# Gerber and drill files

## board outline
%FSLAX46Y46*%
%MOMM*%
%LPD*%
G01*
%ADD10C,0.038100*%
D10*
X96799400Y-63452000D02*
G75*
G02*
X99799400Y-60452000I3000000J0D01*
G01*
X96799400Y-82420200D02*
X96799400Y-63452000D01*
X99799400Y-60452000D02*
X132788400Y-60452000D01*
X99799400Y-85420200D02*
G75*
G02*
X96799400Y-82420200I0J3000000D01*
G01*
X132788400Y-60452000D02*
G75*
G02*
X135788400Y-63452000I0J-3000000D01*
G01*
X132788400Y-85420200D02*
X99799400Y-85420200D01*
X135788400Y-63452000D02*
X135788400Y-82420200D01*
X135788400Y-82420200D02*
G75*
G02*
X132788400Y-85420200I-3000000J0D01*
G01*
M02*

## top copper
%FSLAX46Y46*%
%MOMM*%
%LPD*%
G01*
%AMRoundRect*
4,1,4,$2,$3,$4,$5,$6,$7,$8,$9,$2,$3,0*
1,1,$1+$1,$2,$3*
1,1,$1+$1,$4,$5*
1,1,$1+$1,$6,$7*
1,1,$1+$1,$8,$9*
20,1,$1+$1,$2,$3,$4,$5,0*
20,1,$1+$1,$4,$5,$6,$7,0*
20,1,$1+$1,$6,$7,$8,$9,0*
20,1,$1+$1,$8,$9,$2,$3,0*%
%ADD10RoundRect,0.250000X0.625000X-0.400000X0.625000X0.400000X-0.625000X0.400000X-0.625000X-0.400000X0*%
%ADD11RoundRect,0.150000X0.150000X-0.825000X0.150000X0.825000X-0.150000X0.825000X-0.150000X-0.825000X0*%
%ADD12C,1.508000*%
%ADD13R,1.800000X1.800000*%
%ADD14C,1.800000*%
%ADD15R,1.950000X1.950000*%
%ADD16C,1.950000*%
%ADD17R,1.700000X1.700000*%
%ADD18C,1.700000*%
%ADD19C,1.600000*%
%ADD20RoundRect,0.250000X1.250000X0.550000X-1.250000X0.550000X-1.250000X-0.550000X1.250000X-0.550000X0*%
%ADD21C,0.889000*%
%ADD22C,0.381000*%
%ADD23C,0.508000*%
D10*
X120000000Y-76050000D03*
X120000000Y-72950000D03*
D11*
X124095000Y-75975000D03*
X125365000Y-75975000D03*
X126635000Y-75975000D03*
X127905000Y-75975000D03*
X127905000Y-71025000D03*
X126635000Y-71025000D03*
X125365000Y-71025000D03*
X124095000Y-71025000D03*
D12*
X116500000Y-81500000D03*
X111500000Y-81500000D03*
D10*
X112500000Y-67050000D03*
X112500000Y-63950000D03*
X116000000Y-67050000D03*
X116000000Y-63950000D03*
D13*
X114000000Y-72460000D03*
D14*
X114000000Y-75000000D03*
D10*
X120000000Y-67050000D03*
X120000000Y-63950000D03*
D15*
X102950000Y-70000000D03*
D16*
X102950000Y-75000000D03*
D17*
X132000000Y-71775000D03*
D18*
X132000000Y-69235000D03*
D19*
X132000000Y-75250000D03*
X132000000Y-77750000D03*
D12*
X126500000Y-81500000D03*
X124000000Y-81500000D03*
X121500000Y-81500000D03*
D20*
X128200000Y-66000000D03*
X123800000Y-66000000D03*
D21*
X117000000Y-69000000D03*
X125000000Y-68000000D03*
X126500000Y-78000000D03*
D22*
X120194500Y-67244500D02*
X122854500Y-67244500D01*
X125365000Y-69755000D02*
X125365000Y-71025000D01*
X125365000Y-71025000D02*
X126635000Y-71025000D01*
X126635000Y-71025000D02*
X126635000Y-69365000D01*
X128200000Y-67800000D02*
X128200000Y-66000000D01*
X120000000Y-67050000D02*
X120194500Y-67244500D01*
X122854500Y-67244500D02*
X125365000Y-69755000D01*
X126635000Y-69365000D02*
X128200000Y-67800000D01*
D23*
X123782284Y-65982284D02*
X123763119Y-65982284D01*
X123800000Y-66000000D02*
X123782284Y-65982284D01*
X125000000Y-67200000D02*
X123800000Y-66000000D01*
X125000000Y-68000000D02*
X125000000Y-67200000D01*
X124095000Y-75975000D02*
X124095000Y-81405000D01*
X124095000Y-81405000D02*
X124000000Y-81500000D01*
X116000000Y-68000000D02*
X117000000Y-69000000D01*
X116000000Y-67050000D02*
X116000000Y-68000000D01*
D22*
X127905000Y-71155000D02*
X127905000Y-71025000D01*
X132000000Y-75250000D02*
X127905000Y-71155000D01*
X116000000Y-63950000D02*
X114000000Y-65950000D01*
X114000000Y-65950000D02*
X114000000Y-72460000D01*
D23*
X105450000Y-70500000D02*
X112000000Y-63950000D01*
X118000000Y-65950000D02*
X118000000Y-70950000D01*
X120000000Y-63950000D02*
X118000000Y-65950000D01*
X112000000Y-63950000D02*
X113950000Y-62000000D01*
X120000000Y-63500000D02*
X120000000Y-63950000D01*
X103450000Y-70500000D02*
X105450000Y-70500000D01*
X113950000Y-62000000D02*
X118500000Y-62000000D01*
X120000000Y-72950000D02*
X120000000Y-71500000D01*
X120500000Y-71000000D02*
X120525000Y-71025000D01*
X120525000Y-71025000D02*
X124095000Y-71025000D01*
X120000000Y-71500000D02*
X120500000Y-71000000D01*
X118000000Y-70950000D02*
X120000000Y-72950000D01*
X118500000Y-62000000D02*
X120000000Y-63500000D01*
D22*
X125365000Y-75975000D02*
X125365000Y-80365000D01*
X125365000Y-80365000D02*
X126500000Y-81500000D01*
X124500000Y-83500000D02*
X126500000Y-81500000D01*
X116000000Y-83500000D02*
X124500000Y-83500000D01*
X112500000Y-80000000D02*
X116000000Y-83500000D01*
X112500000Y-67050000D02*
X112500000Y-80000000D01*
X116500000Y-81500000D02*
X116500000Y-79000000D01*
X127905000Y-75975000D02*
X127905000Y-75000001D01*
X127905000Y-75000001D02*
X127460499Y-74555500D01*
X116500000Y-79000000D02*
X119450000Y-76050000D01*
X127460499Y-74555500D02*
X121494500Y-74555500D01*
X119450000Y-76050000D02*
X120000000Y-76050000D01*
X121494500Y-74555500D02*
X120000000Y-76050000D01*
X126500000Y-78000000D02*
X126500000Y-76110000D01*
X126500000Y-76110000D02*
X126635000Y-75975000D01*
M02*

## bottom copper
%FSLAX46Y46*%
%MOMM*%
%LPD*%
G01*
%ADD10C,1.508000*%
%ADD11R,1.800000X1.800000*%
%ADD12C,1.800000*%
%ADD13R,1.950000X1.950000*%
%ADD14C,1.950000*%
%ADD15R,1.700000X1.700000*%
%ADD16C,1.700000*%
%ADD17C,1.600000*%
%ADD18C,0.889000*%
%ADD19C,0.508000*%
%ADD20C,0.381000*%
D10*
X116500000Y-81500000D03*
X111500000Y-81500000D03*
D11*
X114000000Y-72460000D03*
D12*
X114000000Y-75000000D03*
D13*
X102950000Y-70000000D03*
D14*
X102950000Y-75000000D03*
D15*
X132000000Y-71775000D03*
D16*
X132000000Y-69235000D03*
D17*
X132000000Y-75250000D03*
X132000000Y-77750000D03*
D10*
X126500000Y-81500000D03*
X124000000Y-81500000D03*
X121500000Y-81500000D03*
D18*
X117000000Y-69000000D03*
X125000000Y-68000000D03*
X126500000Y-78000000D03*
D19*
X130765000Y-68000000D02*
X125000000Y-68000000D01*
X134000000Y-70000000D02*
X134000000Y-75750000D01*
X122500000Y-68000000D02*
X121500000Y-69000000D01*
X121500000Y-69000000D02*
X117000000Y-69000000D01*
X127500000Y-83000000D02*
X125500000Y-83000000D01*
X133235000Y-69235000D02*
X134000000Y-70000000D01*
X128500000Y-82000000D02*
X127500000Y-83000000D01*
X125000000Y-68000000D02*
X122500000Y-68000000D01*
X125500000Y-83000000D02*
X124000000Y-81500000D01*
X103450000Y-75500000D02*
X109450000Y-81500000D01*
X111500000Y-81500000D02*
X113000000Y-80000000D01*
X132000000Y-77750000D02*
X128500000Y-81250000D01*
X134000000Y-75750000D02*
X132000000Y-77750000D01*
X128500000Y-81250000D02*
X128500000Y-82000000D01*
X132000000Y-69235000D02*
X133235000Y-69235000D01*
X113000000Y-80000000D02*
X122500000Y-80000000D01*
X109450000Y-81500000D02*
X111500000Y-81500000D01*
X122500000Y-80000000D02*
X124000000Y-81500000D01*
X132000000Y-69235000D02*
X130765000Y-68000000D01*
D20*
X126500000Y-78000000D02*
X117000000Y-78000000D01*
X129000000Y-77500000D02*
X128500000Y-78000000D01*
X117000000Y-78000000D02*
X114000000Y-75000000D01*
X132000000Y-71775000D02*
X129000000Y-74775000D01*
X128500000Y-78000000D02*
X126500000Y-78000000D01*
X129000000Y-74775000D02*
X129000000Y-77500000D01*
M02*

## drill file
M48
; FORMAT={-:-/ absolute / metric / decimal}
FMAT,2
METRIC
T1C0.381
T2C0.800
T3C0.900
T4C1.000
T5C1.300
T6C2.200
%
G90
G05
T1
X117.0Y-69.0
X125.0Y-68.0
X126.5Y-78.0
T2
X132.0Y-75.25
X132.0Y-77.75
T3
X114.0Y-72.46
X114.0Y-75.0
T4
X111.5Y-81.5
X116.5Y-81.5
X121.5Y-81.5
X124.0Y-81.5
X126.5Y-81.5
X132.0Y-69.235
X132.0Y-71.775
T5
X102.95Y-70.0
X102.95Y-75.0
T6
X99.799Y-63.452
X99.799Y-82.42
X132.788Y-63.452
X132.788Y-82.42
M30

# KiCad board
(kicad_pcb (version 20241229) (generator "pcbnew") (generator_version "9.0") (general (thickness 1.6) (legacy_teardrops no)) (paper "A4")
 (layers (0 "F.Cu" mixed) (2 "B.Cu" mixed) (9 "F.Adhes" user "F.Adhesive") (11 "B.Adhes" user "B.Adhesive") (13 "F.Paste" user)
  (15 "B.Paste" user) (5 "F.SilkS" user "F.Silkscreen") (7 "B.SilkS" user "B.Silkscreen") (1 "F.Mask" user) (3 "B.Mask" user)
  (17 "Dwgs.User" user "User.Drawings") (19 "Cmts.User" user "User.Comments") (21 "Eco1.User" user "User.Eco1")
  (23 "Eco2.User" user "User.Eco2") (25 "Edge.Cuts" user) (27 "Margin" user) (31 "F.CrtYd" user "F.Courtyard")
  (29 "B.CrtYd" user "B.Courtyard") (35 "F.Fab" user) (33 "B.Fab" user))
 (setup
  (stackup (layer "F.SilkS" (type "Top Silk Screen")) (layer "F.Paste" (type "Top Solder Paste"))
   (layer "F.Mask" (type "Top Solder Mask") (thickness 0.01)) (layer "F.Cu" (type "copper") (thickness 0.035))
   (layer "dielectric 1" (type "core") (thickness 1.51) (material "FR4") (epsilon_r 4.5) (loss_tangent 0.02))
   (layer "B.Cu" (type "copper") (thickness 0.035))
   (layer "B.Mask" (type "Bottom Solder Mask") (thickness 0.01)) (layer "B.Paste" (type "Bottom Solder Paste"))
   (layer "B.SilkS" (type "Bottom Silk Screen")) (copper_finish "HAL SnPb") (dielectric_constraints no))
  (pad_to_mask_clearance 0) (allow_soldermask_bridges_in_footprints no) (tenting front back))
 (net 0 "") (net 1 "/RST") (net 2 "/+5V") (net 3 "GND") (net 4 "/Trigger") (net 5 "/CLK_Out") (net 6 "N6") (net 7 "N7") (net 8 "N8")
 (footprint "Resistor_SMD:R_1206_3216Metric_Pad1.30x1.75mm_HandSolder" (layer "F.Cu") (at 120 74.5 90)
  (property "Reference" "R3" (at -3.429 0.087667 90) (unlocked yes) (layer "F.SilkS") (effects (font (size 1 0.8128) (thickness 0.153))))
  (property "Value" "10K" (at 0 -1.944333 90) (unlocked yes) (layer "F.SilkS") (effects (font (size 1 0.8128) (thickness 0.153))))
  (pad "1" smd roundrect (at -1.55 0 90) (size 1.3 1.75) (layers "F.Cu" "F.Mask" "F.Paste") (roundrect_rratio 0.192308) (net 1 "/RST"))
  (pad "2" smd roundrect (at 1.55 0 90) (size 1.3 1.75) (layers "F.Cu" "F.Mask" "F.Paste") (roundrect_rratio 0.192308) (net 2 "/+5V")))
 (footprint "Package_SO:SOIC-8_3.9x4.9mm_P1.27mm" (layer "F.Cu") (at 126 73.5 90)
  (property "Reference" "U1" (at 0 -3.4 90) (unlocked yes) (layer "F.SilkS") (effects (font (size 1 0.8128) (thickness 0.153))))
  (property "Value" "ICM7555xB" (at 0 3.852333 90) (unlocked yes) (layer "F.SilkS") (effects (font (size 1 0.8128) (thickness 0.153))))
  (pad "1" smd roundrect (at -2.475 -1.905 90) (size 1.95 0.6) (layers "F.Cu" "F.Mask" "F.Paste") (roundrect_rratio 0.25) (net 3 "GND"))
  (pad "2" smd roundrect (at -2.475 -0.635 90) (size 1.95 0.6) (layers "F.Cu" "F.Mask" "F.Paste") (roundrect_rratio 0.25) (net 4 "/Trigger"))
  (pad "3" smd roundrect (at -2.475 0.635 90) (size 1.95 0.6) (layers "F.Cu" "F.Mask" "F.Paste") (roundrect_rratio 0.25) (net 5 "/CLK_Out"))
  (pad "4" smd roundrect (at -2.475 1.905 90) (size 1.95 0.6) (layers "F.Cu" "F.Mask" "F.Paste") (roundrect_rratio 0.25) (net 1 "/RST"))
  (pad "5" smd roundrect (at 2.475 1.905 90) (size 1.95 0.6) (layers "F.Cu" "F.Mask" "F.Paste") (roundrect_rratio 0.25) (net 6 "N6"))
  (pad "6" smd roundrect (at 2.475 0.635 90) (size 1.95 0.6) (layers "F.Cu" "F.Mask" "F.Paste") (roundrect_rratio 0.25) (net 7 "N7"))
  (pad "7" smd roundrect (at 2.475 -0.635 90) (size 1.95 0.6) (layers "F.Cu" "F.Mask" "F.Paste") (roundrect_rratio 0.25) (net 7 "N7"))
  (pad "8" smd roundrect (at 2.475 -1.905 90) (size 1.95 0.6) (layers "F.Cu" "F.Mask" "F.Paste") (roundrect_rratio 0.25) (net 2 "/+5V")))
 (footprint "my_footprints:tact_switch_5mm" (layer "F.Cu") (at 114 81.5 180)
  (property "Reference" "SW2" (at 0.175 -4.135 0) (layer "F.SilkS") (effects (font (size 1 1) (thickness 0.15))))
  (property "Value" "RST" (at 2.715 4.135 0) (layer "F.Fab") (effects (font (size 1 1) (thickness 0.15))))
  (pad "1" thru_hole circle (at -2.5 0 180) (size 1.508 1.508) (drill 1) (layers "*.Cu" "*.Mask") (remove_unused_layers no) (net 1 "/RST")
   (solder_mask_margin 0.102))
  (pad "2" thru_hole circle (at 2.5 0 180) (size 1.508 1.508) (drill 1) (layers "*.Cu" "*.Mask") (remove_unused_layers no) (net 3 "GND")
   (solder_mask_margin 0.102)))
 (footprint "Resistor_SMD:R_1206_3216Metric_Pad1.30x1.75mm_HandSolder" (layer "F.Cu") (at 112.5 65.5 90)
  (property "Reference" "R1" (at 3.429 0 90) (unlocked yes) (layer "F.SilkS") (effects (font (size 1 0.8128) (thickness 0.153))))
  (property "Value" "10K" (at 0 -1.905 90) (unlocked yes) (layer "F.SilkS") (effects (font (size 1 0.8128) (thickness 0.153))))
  (pad "1" smd roundrect (at -1.55 0 90) (size 1.3 1.75) (layers "F.Cu" "F.Mask" "F.Paste") (roundrect_rratio 0.192308) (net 4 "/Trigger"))
  (pad "2" smd roundrect (at 1.55 0 90) (size 1.3 1.75) (layers "F.Cu" "F.Mask" "F.Paste") (roundrect_rratio 0.192308) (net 2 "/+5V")))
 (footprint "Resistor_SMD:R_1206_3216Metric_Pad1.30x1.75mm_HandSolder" (layer "F.Cu") (at 116 65.5 90)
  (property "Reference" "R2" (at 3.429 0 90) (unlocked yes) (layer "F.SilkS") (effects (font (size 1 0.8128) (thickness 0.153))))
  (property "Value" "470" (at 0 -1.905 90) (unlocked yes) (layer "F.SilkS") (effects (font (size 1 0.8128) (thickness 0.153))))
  (pad "1" smd roundrect (at -1.55 0 90) (size 1.3 1.75) (layers "F.Cu" "F.Mask" "F.Paste") (roundrect_rratio 0.192308) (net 3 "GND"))
  (pad "2" smd roundrect (at 1.55 0 90) (size 1.3 1.75) (layers "F.Cu" "F.Mask" "F.Paste") (roundrect_rratio 0.192308) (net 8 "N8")))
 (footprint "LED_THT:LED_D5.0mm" (layer "F.Cu") (at 114 72.46 -90)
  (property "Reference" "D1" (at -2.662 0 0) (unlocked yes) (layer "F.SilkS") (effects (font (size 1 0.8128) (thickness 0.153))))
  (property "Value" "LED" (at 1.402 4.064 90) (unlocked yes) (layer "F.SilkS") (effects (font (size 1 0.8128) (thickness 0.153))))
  (pad "1" thru_hole rect (at 0 0 270) (size 1.8 1.8) (drill 0.9) (layers "*.Cu" "*.Mask") (remove_unused_layers no) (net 8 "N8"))
  (pad "2" thru_hole circle (at 2.54 0 270) (size 1.8 1.8) (drill 0.9) (layers "*.Cu" "*.Mask") (remove_unused_layers no) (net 5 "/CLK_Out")))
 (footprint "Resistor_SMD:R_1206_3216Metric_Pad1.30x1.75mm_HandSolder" (layer "F.Cu") (at 120 65.5 90)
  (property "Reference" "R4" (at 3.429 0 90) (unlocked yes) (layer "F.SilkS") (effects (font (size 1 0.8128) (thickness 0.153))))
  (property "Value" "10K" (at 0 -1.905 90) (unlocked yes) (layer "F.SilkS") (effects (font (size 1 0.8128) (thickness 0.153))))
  (pad "1" smd roundrect (at -1.55 0 90) (size 1.3 1.75) (layers "F.Cu" "F.Mask" "F.Paste") (roundrect_rratio 0.192308) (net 7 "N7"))
  (pad "2" smd roundrect (at 1.55 0 90) (size 1.3 1.75) (layers "F.Cu" "F.Mask" "F.Paste") (roundrect_rratio 0.192308) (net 2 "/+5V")))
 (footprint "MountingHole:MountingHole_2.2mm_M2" (layer "F.Cu") (at 99.7994 63.452)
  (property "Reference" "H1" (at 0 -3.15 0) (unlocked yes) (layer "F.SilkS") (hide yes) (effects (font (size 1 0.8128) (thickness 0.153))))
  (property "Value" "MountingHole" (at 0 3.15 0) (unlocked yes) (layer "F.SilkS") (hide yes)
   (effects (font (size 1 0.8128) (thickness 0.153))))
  (pad "" np_thru_hole circle (at 0 0) (size 2.2 2.2) (drill 2.2) (layers "*.Cu" "*.Mask")))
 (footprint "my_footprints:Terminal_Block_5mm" (layer "F.Cu") (at 102.95 72.5 -90)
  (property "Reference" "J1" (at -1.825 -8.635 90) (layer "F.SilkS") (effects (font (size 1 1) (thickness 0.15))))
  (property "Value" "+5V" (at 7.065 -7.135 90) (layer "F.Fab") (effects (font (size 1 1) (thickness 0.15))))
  (pad "1" thru_hole rect (at -2.5 0 270) (size 1.95 1.95) (drill 1.3) (layers "*.Cu" "*.Mask") (remove_unused_layers no) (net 2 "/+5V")
   (solder_mask_margin 0.102))
  (pad "2" thru_hole circle (at 2.5 0 270) (size 1.95 1.95) (drill 1.3) (layers "*.Cu" "*.Mask") (remove_unused_layers no) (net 3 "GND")
   (solder_mask_margin 0.102)))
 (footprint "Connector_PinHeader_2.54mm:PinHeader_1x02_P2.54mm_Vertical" (layer "F.Cu") (at 132 71.775 180)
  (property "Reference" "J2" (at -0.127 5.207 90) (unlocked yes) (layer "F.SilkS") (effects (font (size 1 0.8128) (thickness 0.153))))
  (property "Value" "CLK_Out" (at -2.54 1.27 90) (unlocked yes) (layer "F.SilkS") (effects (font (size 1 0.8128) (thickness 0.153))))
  (pad "1" thru_hole rect (at 0 0 180) (size 1.7 1.7) (drill 1) (layers "*.Cu" "*.Mask") (remove_unused_layers no) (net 5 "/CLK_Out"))
  (pad "2" thru_hole circle (at 0 2.54 180) (size 1.7 1.7) (drill 1) (layers "*.Cu" "*.Mask") (remove_unused_layers no) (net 3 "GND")))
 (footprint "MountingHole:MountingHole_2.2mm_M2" (layer "F.Cu") (at 132.7884 82.4202)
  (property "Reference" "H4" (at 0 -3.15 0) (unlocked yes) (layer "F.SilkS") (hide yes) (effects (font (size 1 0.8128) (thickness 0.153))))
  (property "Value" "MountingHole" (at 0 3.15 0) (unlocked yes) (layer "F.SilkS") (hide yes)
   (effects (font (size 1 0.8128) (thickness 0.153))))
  (pad "" np_thru_hole circle (at 0 0) (size 2.2 2.2) (drill 2.2) (layers "*.Cu" "*.Mask")))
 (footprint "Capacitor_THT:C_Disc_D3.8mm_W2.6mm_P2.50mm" (layer "F.Cu") (at 132 75.25 -90)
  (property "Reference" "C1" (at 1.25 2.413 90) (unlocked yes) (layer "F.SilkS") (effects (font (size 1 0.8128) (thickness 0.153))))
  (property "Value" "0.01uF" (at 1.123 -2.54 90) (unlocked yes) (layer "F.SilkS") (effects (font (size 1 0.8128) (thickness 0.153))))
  (pad "1" thru_hole circle (at 0 0 270) (size 1.6 1.6) (drill 0.8) (layers "*.Cu" "*.Mask") (remove_unused_layers no) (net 6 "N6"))
  (pad "2" thru_hole circle (at 2.5 0 270) (size 1.6 1.6) (drill 0.8) (layers "*.Cu" "*.Mask") (remove_unused_layers no) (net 3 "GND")))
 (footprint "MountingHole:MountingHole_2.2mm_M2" (layer "F.Cu") (at 132.7884 63.452)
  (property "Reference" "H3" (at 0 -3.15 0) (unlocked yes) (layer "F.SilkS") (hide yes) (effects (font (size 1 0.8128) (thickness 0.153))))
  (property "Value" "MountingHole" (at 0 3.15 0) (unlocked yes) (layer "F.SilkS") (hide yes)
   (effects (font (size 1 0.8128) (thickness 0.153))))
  (pad "" np_thru_hole circle (at 0 0) (size 2.2 2.2) (drill 2.2) (layers "*.Cu" "*.Mask")))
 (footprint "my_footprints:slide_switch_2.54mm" (layer "F.Cu") (at 124 81.5 180)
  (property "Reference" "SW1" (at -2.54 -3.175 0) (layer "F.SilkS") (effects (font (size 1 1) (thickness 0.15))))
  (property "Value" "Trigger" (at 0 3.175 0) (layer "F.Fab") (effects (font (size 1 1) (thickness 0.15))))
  (pad "1" thru_hole circle (at -2.5 0 180) (size 1.508 1.508) (drill 1) (layers "*.Cu" "*.Mask") (remove_unused_layers no)
   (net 4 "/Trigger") (solder_mask_margin 0.102))
  (pad "2" thru_hole circle (at 0 0 180) (size 1.508 1.508) (drill 1) (layers "*.Cu" "*.Mask") (remove_unused_layers no) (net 3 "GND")
   (solder_mask_margin 0.102))
  (pad "3" thru_hole circle (at 2.5 0 180) (size 1.508 1.508) (drill 1) (layers "*.Cu" "*.Mask") (remove_unused_layers no)
   (solder_mask_margin 0.102)))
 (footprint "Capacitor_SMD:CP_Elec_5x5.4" (layer "F.Cu") (at 126 66 180)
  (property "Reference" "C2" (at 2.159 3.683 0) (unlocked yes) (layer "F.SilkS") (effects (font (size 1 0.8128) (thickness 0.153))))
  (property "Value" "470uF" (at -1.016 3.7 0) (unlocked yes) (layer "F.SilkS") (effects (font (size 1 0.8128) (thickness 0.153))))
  (pad "1" smd roundrect (at -2.2 0 180) (size 3 1.6) (layers "F.Cu" "F.Mask" "F.Paste") (roundrect_rratio 0.15625) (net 7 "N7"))
  (pad "2" smd roundrect (at 2.2 0 180) (size 3 1.6) (layers "F.Cu" "F.Mask" "F.Paste") (roundrect_rratio 0.15625) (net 3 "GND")))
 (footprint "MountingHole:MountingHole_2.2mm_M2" (layer "F.Cu") (at 99.7994 82.4202)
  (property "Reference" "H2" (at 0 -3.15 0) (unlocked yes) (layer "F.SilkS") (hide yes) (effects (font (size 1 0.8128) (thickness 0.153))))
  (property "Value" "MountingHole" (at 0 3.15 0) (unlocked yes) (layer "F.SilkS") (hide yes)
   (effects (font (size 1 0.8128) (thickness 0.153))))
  (pad "" np_thru_hole circle (at 0 0) (size 2.2 2.2) (drill 2.2) (layers "*.Cu" "*.Mask")))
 (gr_arc (start 96.7994 63.452) (mid 97.67808 61.33068) (end 99.7994 60.452) (stroke (width 0.0381) (type default)) (layer "Edge.Cuts"))
 (gr_line (start 96.7994 82.4202) (end 96.7994 63.452) (stroke (width 0.0381) (type default)) (layer "Edge.Cuts"))
 (gr_line (start 99.7994 60.452) (end 132.7884 60.452) (stroke (width 0.0381) (type default)) (layer "Edge.Cuts"))
 (gr_arc (start 99.7994 85.4202) (mid 97.67808 84.54152) (end 96.7994 82.4202) (stroke (width 0.0381) (type default)) (layer "Edge.Cuts"))
 (gr_arc (start 132.7884 60.452) (mid 134.90972 61.33068) (end 135.7884 63.452) (stroke (width 0.0381) (type default)) (layer "Edge.Cuts"))
 (gr_line (start 132.7884 85.4202) (end 99.7994 85.4202) (stroke (width 0.0381) (type default)) (layer "Edge.Cuts"))
 (gr_line (start 135.7884 63.452) (end 135.7884 82.4202) (stroke (width 0.0381) (type default)) (layer "Edge.Cuts"))
 (gr_arc (start 135.7884 82.4202) (mid 134.90972 84.54152) (end 132.7884 85.4202) (stroke (width 0.0381) (type default)) (layer "Edge.Cuts"))
 (segment (start 120.1945 67.2445) (end 122.8545 67.2445) (width 0.381) (layer "F.Cu") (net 7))
 (segment (start 125.365 69.755) (end 125.365 71.025) (width 0.381) (layer "F.Cu") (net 7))
 (segment (start 125.365 71.025) (end 126.635 71.025) (width 0.381) (layer "F.Cu") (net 7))
 (segment (start 126.635 71.025) (end 126.635 69.365) (width 0.381) (layer "F.Cu") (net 7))
 (segment (start 128.2 67.8) (end 128.2 66) (width 0.381) (layer "F.Cu") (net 7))
 (segment (start 120 67.05) (end 120.1945 67.2445) (width 0.381) (layer "F.Cu") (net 7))
 (segment (start 122.8545 67.2445) (end 125.365 69.755) (width 0.381) (layer "F.Cu") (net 7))
 (segment (start 126.635 69.365) (end 128.2 67.8) (width 0.381) (layer "F.Cu") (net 7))
 (segment (start 123.782284 65.982284) (end 123.763119 65.982284) (width 0.508) (layer "F.Cu") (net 3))
 (segment (start 123.8 66) (end 123.782284 65.982284) (width 0.508) (layer "F.Cu") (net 3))
 (segment (start 125 67.2) (end 123.8 66) (width 0.508) (layer "F.Cu") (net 3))
 (segment (start 125 68) (end 125 67.2) (width 0.508) (layer "F.Cu") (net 3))
 (segment (start 124.095 75.975) (end 124.095 81.405) (width 0.508) (layer "F.Cu") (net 3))
 (segment (start 124.095 81.405) (end 124 81.5) (width 0.508) (layer "F.Cu") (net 3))
 (segment (start 116 68) (end 117 69) (width 0.508) (layer "F.Cu") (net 3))
 (segment (start 116 67.05) (end 116 68) (width 0.508) (layer "F.Cu") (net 3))
 (via (at 117 69) (size 0.889) (drill 0.381) (layers "F.Cu" "B.Cu") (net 3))
 (via (at 125 68) (size 0.889) (drill 0.381) (layers "F.Cu" "B.Cu") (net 3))
 (segment (start 130.765 68) (end 125 68) (width 0.508) (layer "B.Cu") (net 3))
 (segment (start 134 70) (end 134 75.75) (width 0.508) (layer "B.Cu") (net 3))
 (segment (start 122.5 68) (end 121.5 69) (width 0.508) (layer "B.Cu") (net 3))
 (segment (start 121.5 69) (end 117 69) (width 0.508) (layer "B.Cu") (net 3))
 (segment (start 127.5 83) (end 125.5 83) (width 0.508) (layer "B.Cu") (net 3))
 (segment (start 133.235 69.235) (end 134 70) (width 0.508) (layer "B.Cu") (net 3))
 (segment (start 128.5 82) (end 127.5 83) (width 0.508) (layer "B.Cu") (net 3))
 (segment (start 125 68) (end 122.5 68) (width 0.508) (layer "B.Cu") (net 3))
 (segment (start 125.5 83) (end 124 81.5) (width 0.508) (layer "B.Cu") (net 3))
 (segment (start 103.45 75.5) (end 109.45 81.5) (width 0.508) (layer "B.Cu") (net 3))
 (segment (start 111.5 81.5) (end 113 80) (width 0.508) (layer "B.Cu") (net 3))
 (segment (start 132 77.75) (end 128.5 81.25) (width 0.508) (layer "B.Cu") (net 3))
 (segment (start 134 75.75) (end 132 77.75) (width 0.508) (layer "B.Cu") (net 3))
 (segment (start 128.5 81.25) (end 128.5 82) (width 0.508) (layer "B.Cu") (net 3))
 (segment (start 132 69.235) (end 133.235 69.235) (width 0.508) (layer "B.Cu") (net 3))
 (segment (start 113 80) (end 122.5 80) (width 0.508) (layer "B.Cu") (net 3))
 (segment (start 109.45 81.5) (end 111.5 81.5) (width 0.508) (layer "B.Cu") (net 3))
 (segment (start 122.5 80) (end 124 81.5) (width 0.508) (layer "B.Cu") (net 3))
 (segment (start 132 69.235) (end 130.765 68) (width 0.508) (layer "B.Cu") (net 3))
 (segment (start 127.905 71.155) (end 127.905 71.025) (width 0.381) (layer "F.Cu") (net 6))
 (segment (start 132 75.25) (end 127.905 71.155) (width 0.381) (layer "F.Cu") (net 6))
 (segment (start 116 63.95) (end 114 65.95) (width 0.381) (layer "F.Cu") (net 8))
 (segment (start 114 65.95) (end 114 72.46) (width 0.381) (layer "F.Cu") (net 8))
 (segment (start 105.45 70.5) (end 112 63.95) (width 0.508) (layer "F.Cu") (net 2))
 (segment (start 118 65.95) (end 118 70.95) (width 0.508) (layer "F.Cu") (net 2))
 (segment (start 120 63.95) (end 118 65.95) (width 0.508) (layer "F.Cu") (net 2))
 (segment (start 112 63.95) (end 113.95 62) (width 0.508) (layer "F.Cu") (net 2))
 (segment (start 120 63.5) (end 120 63.95) (width 0.508) (layer "F.Cu") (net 2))
 (segment (start 103.45 70.5) (end 105.45 70.5) (width 0.508) (layer "F.Cu") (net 2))
 (segment (start 113.95 62) (end 118.5 62) (width 0.508) (layer "F.Cu") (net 2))
 (segment (start 120 72.95) (end 120 71.5) (width 0.508) (layer "F.Cu") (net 2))
 (segment (start 120.5 71) (end 120.525 71.025) (width 0.508) (layer "F.Cu") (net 2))
 (segment (start 120.525 71.025) (end 124.095 71.025) (width 0.508) (layer "F.Cu") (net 2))
 (segment (start 120 71.5) (end 120.5 71) (width 0.508) (layer "F.Cu") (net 2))
 (segment (start 118 70.95) (end 120 72.95) (width 0.508) (layer "F.Cu") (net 2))
 (segment (start 118.5 62) (end 120 63.5) (width 0.508) (layer "F.Cu") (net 2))
 (segment (start 125.365 75.975) (end 125.365 80.365) (width 0.381) (layer "F.Cu") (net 4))
 (segment (start 125.365 80.365) (end 126.5 81.5) (width 0.381) (layer "F.Cu") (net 4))
 (segment (start 124.5 83.5) (end 126.5 81.5) (width 0.381) (layer "F.Cu") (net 4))
 (segment (start 116 83.5) (end 124.5 83.5) (width 0.381) (layer "F.Cu") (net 4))
 (segment (start 112.5 80) (end 116 83.5) (width 0.381) (layer "F.Cu") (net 4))
 (segment (start 112.5 67.05) (end 112.5 80) (width 0.381) (layer "F.Cu") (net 4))
 (segment (start 116.5 81.5) (end 116.5 79) (width 0.381) (layer "F.Cu") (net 1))
 (segment (start 127.905 75.975) (end 127.905 75.000001) (width 0.381) (layer "F.Cu") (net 1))
 (segment (start 127.905 75.000001) (end 127.460499 74.5555) (width 0.381) (layer "F.Cu") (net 1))
 (segment (start 116.5 79) (end 119.45 76.05) (width 0.381) (layer "F.Cu") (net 1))
 (segment (start 127.460499 74.5555) (end 121.4945 74.5555) (width 0.381) (layer "F.Cu") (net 1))
 (segment (start 119.45 76.05) (end 120 76.05) (width 0.381) (layer "F.Cu") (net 1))
 (segment (start 121.4945 74.5555) (end 120 76.05) (width 0.381) (layer "F.Cu") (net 1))
 (segment (start 126.5 78) (end 126.5 76.11) (width 0.381) (layer "F.Cu") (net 5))
 (segment (start 126.5 76.11) (end 126.635 75.975) (width 0.381) (layer "F.Cu") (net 5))
 (via (at 126.5 78) (size 0.889) (drill 0.381) (layers "F.Cu" "B.Cu") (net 5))
 (segment (start 126.5 78) (end 117 78) (width 0.381) (layer "B.Cu") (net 5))
 (segment (start 129 77.5) (end 128.5 78) (width 0.381) (layer "B.Cu") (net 5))
 (segment (start 117 78) (end 114 75) (width 0.381) (layer "B.Cu") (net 5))
 (segment (start 132 71.775) (end 129 74.775) (width 0.381) (layer "B.Cu") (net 5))
 (segment (start 128.5 78) (end 126.5 78) (width 0.381) (layer "B.Cu") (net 5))
 (segment (start 129 74.775) (end 129 77.5) (width 0.381) (layer "B.Cu") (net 5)))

